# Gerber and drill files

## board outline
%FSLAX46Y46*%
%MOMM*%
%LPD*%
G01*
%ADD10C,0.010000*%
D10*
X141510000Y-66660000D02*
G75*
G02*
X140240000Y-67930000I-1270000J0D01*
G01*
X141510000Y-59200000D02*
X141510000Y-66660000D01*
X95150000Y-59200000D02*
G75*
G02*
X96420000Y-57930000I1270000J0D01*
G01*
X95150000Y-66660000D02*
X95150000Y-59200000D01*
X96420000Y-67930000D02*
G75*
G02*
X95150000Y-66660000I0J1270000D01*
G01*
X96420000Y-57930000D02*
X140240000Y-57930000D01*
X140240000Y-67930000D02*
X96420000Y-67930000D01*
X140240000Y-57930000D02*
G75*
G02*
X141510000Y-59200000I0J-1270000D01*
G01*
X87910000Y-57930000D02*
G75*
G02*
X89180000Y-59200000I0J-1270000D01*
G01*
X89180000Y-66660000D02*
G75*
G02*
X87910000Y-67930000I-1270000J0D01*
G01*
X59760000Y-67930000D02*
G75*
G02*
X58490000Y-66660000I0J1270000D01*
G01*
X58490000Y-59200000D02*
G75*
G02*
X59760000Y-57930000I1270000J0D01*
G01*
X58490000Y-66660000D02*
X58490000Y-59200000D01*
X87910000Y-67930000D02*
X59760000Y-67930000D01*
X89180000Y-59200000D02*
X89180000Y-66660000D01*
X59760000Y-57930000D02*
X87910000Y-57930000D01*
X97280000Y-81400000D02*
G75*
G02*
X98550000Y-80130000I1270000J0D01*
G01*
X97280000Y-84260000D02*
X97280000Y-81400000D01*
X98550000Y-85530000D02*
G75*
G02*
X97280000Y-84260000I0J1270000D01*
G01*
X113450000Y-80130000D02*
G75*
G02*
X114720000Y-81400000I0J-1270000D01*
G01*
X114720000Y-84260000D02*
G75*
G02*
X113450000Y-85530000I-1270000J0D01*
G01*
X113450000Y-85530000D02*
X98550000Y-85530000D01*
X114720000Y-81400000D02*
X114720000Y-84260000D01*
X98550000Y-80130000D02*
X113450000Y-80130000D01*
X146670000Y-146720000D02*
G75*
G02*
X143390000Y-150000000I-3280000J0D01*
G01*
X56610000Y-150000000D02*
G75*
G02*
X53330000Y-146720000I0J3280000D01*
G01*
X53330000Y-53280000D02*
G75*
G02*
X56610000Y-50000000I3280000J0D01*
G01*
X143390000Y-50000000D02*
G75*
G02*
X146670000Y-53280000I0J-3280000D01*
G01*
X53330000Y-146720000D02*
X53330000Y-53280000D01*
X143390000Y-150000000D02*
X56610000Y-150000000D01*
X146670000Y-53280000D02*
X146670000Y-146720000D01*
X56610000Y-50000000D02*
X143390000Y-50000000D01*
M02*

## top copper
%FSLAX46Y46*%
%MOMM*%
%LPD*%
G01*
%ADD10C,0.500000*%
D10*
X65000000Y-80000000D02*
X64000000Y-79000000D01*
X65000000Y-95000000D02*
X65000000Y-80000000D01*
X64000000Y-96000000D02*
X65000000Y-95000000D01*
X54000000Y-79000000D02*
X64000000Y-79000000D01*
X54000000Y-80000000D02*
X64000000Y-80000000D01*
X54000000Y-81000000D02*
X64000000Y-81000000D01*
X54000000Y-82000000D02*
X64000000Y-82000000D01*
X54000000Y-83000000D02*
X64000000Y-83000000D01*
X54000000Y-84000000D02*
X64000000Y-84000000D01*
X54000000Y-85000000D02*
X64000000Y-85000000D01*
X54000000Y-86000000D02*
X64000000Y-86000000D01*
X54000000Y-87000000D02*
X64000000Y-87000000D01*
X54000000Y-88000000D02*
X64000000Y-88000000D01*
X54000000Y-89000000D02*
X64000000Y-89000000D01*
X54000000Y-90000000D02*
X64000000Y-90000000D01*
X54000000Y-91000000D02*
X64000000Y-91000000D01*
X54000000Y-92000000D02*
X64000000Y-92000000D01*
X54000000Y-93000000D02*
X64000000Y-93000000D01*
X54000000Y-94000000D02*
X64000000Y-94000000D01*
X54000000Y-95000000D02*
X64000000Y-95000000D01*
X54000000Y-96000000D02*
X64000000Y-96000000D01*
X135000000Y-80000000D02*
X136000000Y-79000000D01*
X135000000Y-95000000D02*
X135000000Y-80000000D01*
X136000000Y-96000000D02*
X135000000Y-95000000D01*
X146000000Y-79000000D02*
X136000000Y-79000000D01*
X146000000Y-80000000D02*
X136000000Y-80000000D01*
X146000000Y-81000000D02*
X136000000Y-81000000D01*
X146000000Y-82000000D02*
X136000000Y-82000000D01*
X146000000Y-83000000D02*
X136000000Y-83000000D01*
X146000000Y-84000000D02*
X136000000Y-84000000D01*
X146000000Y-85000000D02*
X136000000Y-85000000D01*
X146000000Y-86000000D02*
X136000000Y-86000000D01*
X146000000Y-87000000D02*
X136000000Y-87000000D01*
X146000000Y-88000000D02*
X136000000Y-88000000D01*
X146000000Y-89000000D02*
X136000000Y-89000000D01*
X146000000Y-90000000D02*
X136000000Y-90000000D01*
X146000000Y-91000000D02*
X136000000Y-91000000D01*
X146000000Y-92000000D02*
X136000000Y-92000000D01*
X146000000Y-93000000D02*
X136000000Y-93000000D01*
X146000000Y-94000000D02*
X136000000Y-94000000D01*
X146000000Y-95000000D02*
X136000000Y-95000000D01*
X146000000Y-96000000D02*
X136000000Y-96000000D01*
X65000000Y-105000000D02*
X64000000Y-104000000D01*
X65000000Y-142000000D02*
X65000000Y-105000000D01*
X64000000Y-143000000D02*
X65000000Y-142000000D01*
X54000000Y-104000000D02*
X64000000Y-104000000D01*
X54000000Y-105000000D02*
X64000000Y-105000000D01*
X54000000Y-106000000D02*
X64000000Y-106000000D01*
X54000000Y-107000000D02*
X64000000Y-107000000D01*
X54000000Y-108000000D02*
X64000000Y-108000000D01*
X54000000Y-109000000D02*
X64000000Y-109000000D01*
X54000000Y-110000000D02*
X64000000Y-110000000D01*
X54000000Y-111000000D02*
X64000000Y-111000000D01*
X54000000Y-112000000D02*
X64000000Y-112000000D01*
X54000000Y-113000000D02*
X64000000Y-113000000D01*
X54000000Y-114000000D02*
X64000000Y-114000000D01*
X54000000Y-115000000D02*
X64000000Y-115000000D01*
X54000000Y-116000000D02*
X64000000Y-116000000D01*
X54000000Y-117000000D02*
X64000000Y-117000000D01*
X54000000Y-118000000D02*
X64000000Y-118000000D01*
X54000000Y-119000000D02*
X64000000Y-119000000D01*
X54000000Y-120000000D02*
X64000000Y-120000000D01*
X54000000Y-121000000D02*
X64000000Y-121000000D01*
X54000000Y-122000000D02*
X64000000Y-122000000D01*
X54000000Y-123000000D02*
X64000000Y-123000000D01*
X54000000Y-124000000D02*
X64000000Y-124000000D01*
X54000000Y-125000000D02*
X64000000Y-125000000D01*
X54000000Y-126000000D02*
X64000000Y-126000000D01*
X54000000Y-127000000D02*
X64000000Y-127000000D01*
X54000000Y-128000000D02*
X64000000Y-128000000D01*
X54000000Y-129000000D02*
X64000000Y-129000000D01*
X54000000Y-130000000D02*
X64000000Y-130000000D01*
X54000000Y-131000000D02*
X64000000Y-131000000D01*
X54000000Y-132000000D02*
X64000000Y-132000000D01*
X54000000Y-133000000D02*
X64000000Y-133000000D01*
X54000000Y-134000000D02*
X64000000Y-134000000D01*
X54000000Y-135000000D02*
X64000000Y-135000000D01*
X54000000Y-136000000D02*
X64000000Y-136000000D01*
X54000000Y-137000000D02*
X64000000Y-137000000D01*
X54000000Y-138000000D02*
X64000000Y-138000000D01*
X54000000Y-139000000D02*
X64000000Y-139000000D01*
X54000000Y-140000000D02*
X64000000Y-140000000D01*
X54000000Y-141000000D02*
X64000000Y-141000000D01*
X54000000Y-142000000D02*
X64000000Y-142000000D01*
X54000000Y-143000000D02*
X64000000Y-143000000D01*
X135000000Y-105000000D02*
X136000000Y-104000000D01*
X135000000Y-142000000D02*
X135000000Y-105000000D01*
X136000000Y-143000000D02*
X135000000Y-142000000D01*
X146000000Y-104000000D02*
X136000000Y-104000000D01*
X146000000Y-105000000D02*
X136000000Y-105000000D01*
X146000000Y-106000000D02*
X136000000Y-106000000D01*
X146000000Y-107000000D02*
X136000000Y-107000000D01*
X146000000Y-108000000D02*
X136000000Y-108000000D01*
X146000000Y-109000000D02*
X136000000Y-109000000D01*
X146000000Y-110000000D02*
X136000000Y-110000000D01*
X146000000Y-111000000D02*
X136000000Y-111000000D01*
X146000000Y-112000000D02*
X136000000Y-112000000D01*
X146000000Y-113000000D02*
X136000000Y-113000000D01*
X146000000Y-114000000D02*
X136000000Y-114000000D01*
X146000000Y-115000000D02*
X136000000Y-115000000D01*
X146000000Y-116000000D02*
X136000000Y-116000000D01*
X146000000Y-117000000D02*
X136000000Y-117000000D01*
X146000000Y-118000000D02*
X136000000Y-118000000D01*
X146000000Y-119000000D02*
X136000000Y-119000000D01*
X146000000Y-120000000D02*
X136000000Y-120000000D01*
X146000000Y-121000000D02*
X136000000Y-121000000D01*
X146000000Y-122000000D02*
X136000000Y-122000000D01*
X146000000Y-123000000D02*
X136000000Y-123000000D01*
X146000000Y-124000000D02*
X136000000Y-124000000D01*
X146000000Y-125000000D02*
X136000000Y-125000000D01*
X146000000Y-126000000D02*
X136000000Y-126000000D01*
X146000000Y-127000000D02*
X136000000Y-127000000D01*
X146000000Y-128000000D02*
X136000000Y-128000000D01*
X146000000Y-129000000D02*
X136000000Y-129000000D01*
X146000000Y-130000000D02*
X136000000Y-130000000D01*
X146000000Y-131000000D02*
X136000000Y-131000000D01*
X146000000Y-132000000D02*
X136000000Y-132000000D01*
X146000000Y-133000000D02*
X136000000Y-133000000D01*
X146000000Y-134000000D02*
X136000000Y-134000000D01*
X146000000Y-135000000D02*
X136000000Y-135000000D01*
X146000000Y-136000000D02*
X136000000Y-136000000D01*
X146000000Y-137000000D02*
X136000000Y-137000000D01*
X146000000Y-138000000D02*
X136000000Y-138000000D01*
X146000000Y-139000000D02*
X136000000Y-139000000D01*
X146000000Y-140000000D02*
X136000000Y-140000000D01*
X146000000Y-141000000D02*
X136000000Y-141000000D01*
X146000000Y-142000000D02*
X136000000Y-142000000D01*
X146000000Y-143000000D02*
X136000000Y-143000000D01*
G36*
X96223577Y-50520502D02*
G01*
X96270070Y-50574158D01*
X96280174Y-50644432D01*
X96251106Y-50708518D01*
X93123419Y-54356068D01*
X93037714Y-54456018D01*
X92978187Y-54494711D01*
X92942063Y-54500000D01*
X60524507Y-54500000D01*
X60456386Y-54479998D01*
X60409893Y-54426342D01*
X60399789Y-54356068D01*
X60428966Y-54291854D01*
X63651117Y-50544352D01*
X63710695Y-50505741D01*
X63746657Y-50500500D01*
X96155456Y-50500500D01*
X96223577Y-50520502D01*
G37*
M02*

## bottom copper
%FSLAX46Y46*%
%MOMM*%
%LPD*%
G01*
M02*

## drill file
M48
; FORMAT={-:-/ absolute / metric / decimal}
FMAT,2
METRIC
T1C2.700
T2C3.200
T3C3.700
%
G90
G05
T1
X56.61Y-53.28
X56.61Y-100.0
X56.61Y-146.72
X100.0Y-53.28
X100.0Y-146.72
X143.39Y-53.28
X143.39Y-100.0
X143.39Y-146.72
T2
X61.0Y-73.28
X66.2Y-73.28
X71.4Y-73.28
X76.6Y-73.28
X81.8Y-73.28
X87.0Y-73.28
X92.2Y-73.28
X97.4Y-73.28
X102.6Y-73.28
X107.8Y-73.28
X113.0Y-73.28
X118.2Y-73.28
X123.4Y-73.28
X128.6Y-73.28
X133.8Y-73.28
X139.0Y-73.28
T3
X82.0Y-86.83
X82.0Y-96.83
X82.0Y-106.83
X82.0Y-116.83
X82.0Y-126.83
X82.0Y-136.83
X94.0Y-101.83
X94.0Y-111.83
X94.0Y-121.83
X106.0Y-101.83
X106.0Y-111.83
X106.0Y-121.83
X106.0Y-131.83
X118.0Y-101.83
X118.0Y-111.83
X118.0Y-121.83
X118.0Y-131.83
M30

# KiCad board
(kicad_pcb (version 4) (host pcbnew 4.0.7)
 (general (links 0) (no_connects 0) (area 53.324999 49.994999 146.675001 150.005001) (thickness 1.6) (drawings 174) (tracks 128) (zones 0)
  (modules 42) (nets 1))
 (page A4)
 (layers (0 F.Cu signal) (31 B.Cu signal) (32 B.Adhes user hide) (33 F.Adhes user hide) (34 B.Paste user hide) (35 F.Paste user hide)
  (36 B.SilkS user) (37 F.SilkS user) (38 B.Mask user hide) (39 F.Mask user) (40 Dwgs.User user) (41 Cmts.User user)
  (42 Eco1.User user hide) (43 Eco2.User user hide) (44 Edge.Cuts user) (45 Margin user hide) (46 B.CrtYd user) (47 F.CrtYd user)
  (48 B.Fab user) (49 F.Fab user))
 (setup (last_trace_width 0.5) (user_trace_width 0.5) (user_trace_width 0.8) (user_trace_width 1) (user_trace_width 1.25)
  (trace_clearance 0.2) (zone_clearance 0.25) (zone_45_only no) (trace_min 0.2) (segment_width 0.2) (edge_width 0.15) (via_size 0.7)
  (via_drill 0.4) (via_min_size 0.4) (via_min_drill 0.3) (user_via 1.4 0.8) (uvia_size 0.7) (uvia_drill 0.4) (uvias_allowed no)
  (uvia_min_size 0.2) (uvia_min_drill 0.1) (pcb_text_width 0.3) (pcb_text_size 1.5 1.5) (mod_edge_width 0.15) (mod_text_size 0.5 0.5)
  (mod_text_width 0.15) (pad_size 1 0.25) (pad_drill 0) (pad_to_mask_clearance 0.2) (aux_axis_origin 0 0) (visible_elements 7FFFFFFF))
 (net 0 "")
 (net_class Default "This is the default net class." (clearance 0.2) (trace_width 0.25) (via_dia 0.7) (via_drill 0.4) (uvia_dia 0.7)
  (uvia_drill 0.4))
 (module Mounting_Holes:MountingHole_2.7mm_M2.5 (layer F.Cu) (at 143.39 146.72)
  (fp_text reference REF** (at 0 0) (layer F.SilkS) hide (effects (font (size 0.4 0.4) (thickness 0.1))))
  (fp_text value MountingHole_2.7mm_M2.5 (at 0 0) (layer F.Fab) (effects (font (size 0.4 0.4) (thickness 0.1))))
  (pad 1 np_thru_hole circle (at 0 0) (size 2.7 2.7) (drill 2.7) (layers *.Cu *.Mask)))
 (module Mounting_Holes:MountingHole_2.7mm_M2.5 (layer F.Cu) (at 100 146.72)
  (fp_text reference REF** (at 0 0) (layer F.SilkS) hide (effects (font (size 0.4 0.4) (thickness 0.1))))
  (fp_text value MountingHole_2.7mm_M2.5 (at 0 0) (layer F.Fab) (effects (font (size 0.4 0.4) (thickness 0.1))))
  (pad 1 np_thru_hole circle (at 0 0) (size 2.7 2.7) (drill 2.7) (layers *.Cu *.Mask)))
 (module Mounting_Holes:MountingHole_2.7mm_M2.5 (layer F.Cu) (at 56.61 146.72)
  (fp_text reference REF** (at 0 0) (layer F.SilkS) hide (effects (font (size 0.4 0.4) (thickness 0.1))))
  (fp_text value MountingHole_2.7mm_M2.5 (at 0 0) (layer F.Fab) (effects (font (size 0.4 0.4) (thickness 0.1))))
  (pad 1 np_thru_hole circle (at 0 0) (size 2.7 2.7) (drill 2.7) (layers *.Cu *.Mask)))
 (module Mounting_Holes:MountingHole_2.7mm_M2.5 (layer F.Cu) (at 143.39 100)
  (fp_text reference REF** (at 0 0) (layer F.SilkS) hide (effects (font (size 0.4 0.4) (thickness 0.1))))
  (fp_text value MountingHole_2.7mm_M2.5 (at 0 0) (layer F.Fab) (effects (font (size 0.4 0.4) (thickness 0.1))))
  (pad 1 np_thru_hole circle (at 0 0) (size 2.7 2.7) (drill 2.7) (layers *.Cu *.Mask)))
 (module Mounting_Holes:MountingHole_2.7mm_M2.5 (layer F.Cu) (at 56.61 100)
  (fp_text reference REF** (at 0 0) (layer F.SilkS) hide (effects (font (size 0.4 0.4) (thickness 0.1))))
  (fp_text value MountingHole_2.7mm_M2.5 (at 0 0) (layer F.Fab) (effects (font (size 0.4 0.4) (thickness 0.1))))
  (pad 1 np_thru_hole circle (at 0 0) (size 2.7 2.7) (drill 2.7) (layers *.Cu *.Mask)))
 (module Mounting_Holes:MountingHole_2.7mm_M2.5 (layer F.Cu) (at 143.39 53.28)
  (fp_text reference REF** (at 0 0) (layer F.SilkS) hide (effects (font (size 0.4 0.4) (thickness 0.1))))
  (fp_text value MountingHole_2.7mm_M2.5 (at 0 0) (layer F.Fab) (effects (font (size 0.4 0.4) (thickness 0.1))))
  (pad 1 np_thru_hole circle (at 0 0) (size 2.7 2.7) (drill 2.7) (layers *.Cu *.Mask)))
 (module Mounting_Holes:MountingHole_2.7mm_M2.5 (layer F.Cu) (at 100 53.28)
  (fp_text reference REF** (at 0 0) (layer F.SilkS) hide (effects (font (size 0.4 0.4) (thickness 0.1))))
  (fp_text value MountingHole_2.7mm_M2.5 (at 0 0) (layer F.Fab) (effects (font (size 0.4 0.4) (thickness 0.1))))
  (pad 1 np_thru_hole circle (at 0 0) (size 2.7 2.7) (drill 2.7) (layers *.Cu *.Mask)))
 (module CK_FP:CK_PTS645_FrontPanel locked (layer F.Cu) (at 82 136.83)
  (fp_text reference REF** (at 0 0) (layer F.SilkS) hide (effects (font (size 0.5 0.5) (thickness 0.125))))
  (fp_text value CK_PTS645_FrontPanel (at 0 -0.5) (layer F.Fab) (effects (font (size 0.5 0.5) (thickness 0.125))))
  (pad "" np_thru_hole circle (at 0 0) (size 3.7 3.7) (drill 3.7) (layers *.Cu *.Mask)))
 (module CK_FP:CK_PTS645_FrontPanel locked (layer F.Cu) (at 82 86.83)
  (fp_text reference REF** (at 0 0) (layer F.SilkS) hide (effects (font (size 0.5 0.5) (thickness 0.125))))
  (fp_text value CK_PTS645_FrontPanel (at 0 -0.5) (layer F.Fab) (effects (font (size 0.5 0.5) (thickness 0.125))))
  (pad "" np_thru_hole circle (at 0 0) (size 3.7 3.7) (drill 3.7) (layers *.Cu *.Mask)))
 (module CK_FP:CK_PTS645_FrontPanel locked (layer F.Cu) (at 82 96.83)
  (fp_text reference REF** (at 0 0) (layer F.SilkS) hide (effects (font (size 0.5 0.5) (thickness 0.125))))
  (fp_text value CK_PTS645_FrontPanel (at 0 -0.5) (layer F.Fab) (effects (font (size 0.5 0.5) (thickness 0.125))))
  (pad "" np_thru_hole circle (at 0 0) (size 3.7 3.7) (drill 3.7) (layers *.Cu *.Mask)))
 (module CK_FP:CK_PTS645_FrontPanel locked (layer F.Cu) (at 82 106.83)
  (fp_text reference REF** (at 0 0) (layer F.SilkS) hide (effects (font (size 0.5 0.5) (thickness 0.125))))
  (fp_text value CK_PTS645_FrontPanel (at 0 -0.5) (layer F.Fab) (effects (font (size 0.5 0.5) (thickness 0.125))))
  (pad "" np_thru_hole circle (at 0 0) (size 3.7 3.7) (drill 3.7) (layers *.Cu *.Mask)))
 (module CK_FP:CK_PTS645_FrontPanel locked (layer F.Cu) (at 82 116.83)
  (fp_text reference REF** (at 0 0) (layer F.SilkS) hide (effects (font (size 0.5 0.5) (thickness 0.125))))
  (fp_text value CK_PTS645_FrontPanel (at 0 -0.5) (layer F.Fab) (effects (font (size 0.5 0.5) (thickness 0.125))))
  (pad "" np_thru_hole circle (at 0 0) (size 3.7 3.7) (drill 3.7) (layers *.Cu *.Mask)))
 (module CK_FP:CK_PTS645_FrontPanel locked (layer F.Cu) (at 82 126.83)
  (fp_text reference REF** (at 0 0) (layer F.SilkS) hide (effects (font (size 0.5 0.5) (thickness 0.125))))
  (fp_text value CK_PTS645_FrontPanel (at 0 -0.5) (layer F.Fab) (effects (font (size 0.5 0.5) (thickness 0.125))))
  (pad "" np_thru_hole circle (at 0 0) (size 3.7 3.7) (drill 3.7) (layers *.Cu *.Mask)))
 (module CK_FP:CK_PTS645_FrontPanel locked (layer F.Cu) (at 106 131.83)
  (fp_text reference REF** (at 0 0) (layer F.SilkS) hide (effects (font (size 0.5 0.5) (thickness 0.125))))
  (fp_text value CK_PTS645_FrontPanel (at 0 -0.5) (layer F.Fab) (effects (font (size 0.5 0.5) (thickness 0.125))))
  (pad "" np_thru_hole circle (at 0 0) (size 3.7 3.7) (drill 3.7) (layers *.Cu *.Mask)))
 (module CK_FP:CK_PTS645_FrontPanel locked (layer F.Cu) (at 118 131.83)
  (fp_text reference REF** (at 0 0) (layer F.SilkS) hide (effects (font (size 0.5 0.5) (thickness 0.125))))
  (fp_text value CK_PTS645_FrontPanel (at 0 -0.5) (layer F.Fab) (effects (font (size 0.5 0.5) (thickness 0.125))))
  (pad "" np_thru_hole circle (at 0 0) (size 3.7 3.7) (drill 3.7) (layers *.Cu *.Mask)))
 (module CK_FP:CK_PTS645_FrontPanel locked (layer F.Cu) (at 94 121.83)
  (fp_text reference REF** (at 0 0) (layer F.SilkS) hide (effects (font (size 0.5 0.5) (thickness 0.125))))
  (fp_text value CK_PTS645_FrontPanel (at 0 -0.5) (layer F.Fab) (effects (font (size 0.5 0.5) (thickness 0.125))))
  (pad "" np_thru_hole circle (at 0 0) (size 3.7 3.7) (drill 3.7) (layers *.Cu *.Mask)))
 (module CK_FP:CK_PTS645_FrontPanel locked (layer F.Cu) (at 106 121.83)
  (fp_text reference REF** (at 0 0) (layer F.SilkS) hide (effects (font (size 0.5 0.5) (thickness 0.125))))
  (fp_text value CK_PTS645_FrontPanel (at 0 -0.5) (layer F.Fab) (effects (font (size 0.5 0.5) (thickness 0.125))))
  (pad "" np_thru_hole circle (at 0 0) (size 3.7 3.7) (drill 3.7) (layers *.Cu *.Mask)))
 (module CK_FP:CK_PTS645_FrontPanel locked (layer F.Cu) (at 118 121.83)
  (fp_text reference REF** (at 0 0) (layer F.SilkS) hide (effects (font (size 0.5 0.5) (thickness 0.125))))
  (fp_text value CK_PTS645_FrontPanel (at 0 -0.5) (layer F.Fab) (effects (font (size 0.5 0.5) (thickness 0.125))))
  (pad "" np_thru_hole circle (at 0 0) (size 3.7 3.7) (drill 3.7) (layers *.Cu *.Mask)))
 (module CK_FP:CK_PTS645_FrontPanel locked (layer F.Cu) (at 94 111.83)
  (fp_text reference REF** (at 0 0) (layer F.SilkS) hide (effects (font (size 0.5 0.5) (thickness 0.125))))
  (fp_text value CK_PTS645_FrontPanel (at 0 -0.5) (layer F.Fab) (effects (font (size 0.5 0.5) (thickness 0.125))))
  (pad "" np_thru_hole circle (at 0 0) (size 3.7 3.7) (drill 3.7) (layers *.Cu *.Mask)))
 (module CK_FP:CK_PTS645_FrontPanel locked (layer F.Cu) (at 106 111.83)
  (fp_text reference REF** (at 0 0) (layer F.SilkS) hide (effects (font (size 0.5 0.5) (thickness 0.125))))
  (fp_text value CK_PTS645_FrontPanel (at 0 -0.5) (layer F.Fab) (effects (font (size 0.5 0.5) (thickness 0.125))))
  (pad "" np_thru_hole circle (at 0 0) (size 3.7 3.7) (drill 3.7) (layers *.Cu *.Mask)))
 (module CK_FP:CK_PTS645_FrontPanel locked (layer F.Cu) (at 118 111.83)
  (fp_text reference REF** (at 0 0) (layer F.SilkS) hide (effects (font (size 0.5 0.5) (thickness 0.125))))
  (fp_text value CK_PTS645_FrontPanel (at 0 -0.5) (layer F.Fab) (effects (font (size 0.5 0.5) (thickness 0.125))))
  (pad "" np_thru_hole circle (at 0 0) (size 3.7 3.7) (drill 3.7) (layers *.Cu *.Mask)))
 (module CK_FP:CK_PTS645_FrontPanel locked (layer F.Cu) (at 94 101.83)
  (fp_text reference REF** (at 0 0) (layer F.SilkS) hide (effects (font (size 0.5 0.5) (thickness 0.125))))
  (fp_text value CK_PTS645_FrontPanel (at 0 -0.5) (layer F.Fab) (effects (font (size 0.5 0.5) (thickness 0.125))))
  (pad "" np_thru_hole circle (at 0 0) (size 3.7 3.7) (drill 3.7) (layers *.Cu *.Mask)))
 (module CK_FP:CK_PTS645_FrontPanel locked (layer F.Cu) (at 106 101.83)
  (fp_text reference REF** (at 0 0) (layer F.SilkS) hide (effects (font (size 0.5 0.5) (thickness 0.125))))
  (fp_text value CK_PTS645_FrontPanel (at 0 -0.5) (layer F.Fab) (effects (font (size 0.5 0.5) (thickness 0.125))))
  (pad "" np_thru_hole circle (at 0 0) (size 3.7 3.7) (drill 3.7) (layers *.Cu *.Mask)))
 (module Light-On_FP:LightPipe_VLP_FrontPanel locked (layer F.Cu) (at 61 73.28)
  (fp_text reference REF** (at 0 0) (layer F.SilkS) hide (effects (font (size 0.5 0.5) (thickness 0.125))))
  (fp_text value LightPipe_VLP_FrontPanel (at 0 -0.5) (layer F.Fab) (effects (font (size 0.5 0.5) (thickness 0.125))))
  (pad "" np_thru_hole circle (at 0 0) (size 3.2 3.2) (drill 3.2) (layers *.Cu *.Mask)))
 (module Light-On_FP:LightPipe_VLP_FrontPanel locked (layer F.Cu) (at 66.2 73.28)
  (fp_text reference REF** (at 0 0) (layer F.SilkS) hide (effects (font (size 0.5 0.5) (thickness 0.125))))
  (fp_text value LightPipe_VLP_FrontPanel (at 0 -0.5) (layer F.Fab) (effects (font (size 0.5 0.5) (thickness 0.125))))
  (pad "" np_thru_hole circle (at 0 0) (size 3.2 3.2) (drill 3.2) (layers *.Cu *.Mask)))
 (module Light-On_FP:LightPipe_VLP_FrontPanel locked (layer F.Cu) (at 71.4 73.28)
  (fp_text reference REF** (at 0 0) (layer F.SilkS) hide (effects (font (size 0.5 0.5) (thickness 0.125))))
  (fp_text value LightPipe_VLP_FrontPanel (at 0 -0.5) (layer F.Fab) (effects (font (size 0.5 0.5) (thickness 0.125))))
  (pad "" np_thru_hole circle (at 0 0) (size 3.2 3.2) (drill 3.2) (layers *.Cu *.Mask)))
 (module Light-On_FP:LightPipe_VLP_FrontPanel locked (layer F.Cu) (at 76.6 73.28)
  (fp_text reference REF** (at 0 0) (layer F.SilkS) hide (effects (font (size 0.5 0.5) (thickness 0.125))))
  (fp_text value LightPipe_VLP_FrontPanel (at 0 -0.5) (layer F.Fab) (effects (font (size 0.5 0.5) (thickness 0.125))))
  (pad "" np_thru_hole circle (at 0 0) (size 3.2 3.2) (drill 3.2) (layers *.Cu *.Mask)))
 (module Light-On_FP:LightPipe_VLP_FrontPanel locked (layer F.Cu) (at 81.8 73.28)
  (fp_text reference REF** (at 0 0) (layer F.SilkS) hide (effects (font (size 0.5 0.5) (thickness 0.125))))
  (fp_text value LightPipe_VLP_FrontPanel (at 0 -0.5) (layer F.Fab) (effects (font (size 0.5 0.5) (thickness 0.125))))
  (pad "" np_thru_hole circle (at 0 0) (size 3.2 3.2) (drill 3.2) (layers *.Cu *.Mask)))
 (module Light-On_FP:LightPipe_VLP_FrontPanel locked (layer F.Cu) (at 87 73.28)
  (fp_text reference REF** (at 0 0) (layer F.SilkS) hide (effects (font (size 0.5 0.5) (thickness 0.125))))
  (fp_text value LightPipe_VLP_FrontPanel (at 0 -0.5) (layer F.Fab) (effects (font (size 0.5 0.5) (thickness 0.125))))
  (pad "" np_thru_hole circle (at 0 0) (size 3.2 3.2) (drill 3.2) (layers *.Cu *.Mask)))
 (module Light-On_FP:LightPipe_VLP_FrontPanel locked (layer F.Cu) (at 92.2 73.28)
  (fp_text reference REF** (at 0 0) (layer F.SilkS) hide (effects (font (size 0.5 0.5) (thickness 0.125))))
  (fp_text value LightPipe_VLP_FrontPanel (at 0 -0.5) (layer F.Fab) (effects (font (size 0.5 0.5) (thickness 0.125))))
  (pad "" np_thru_hole circle (at 0 0) (size 3.2 3.2) (drill 3.2) (layers *.Cu *.Mask)))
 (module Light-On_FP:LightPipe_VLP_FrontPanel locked (layer F.Cu) (at 97.4 73.28)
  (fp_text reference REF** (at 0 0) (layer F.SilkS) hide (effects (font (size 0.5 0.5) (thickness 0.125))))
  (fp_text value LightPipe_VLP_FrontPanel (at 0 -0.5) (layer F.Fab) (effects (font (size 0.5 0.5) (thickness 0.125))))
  (pad "" np_thru_hole circle (at 0 0) (size 3.2 3.2) (drill 3.2) (layers *.Cu *.Mask)))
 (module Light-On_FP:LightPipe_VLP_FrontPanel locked (layer F.Cu) (at 102.6 73.28)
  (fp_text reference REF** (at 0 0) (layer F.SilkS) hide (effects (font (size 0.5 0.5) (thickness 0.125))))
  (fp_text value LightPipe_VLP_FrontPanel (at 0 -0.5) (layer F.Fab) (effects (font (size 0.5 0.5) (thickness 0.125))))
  (pad "" np_thru_hole circle (at 0 0) (size 3.2 3.2) (drill 3.2) (layers *.Cu *.Mask)))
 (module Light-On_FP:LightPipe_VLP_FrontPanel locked (layer F.Cu) (at 107.8 73.28)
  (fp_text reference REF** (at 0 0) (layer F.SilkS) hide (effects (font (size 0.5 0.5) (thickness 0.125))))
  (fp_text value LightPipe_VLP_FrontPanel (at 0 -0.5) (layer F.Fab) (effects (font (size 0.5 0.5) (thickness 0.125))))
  (pad "" np_thru_hole circle (at 0 0) (size 3.2 3.2) (drill 3.2) (layers *.Cu *.Mask)))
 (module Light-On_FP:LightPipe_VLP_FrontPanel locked (layer F.Cu) (at 113 73.28)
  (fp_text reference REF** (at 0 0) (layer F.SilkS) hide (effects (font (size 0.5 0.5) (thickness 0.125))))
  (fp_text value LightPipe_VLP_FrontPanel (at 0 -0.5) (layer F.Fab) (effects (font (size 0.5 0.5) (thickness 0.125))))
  (pad "" np_thru_hole circle (at 0 0) (size 3.2 3.2) (drill 3.2) (layers *.Cu *.Mask)))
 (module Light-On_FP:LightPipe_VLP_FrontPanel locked (layer F.Cu) (at 118.2 73.28)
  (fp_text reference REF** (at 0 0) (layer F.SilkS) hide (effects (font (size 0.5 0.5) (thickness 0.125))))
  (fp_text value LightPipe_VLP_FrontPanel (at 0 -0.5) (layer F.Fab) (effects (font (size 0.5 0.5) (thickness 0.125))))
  (pad "" np_thru_hole circle (at 0 0) (size 3.2 3.2) (drill 3.2) (layers *.Cu *.Mask)))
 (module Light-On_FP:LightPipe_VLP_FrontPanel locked (layer F.Cu) (at 123.4 73.28)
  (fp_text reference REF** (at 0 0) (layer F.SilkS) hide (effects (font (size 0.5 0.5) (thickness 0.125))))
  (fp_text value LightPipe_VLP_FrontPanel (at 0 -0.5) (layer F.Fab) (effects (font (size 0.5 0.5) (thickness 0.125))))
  (pad "" np_thru_hole circle (at 0 0) (size 3.2 3.2) (drill 3.2) (layers *.Cu *.Mask)))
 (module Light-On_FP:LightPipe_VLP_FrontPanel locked (layer F.Cu) (at 128.6 73.28)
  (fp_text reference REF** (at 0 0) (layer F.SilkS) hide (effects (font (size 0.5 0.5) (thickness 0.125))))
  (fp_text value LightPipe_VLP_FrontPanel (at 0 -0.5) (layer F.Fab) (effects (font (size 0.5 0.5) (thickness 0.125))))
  (pad "" np_thru_hole circle (at 0 0) (size 3.2 3.2) (drill 3.2) (layers *.Cu *.Mask)))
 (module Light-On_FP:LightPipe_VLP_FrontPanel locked (layer F.Cu) (at 133.8 73.28)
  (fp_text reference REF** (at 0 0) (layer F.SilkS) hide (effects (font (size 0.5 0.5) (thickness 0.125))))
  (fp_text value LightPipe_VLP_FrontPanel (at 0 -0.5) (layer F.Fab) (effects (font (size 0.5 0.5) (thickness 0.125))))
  (pad "" np_thru_hole circle (at 0 0) (size 3.2 3.2) (drill 3.2) (layers *.Cu *.Mask)))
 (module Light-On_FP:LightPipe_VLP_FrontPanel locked (layer F.Cu) (at 139 73.28)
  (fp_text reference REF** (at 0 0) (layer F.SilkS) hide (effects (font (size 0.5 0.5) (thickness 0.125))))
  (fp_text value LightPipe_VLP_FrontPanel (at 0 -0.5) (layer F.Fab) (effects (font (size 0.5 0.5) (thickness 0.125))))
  (pad "" np_thru_hole circle (at 0 0) (size 3.2 3.2) (drill 3.2) (layers *.Cu *.Mask)))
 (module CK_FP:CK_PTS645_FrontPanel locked (layer F.Cu) (at 118 101.83)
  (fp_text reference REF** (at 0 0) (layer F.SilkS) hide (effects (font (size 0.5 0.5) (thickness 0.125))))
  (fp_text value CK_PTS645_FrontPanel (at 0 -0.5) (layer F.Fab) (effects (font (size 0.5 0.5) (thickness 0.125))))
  (pad "" np_thru_hole circle (at 0 0) (size 3.7 3.7) (drill 3.7) (layers *.Cu *.Mask)))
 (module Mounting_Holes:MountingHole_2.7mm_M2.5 (layer F.Cu) (at 56.61 53.28)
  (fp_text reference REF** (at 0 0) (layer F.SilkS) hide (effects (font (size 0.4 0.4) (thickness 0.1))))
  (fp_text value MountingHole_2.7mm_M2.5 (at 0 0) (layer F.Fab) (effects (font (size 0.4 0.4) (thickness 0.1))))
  (pad 1 np_thru_hole circle (at 0 0) (size 2.7 2.7) (drill 2.7) (layers *.Cu *.Mask)))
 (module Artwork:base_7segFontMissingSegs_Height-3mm (layer F.Cu) (at 72.19 52.37)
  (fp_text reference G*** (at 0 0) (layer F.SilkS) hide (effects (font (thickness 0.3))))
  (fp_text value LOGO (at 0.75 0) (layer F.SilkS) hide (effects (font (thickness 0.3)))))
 (gr_arc (start 140.24 66.66) (end 141.51 66.66) (angle 90) (layer Edge.Cuts) (width 0.01))
 (gr_line (start 141.51 59.2) (end 141.51 66.66) (layer Edge.Cuts) (width 0.01))
 (gr_arc (start 96.42 59.2) (end 95.15 59.2) (angle 90) (layer Edge.Cuts) (width 0.01))
 (gr_line (start 95.15 66.66) (end 95.15 59.2) (layer Edge.Cuts) (width 0.01))
 (gr_arc (start 96.42 66.66) (end 96.42 67.93) (angle 90) (layer Edge.Cuts) (width 0.01))
 (gr_line (start 96.42 57.93) (end 140.24 57.93) (layer Edge.Cuts) (width 0.01))
 (gr_line (start 140.24 67.93) (end 96.42 67.93) (layer Edge.Cuts) (width 0.01))
 (gr_arc (start 140.24 59.2) (end 140.24 57.93) (angle 90) (layer Edge.Cuts) (width 0.01))
 (gr_arc (start 87.91 59.2) (end 87.91 57.93) (angle 90) (layer Edge.Cuts) (width 0.01))
 (gr_arc (start 87.91 66.66) (end 89.18 66.66) (angle 90) (layer Edge.Cuts) (width 0.01))
 (gr_arc (start 59.76 66.66) (end 59.76 67.93) (angle 90) (layer Edge.Cuts) (width 0.01))
 (gr_arc (start 59.76 59.2) (end 58.49 59.2) (angle 90) (layer Edge.Cuts) (width 0.01))
 (gr_line (start 58.49 66.66) (end 58.49 59.2) (layer Edge.Cuts) (width 0.01))
 (gr_line (start 87.91 67.93) (end 59.76 67.93) (layer Edge.Cuts) (width 0.01))
 (gr_line (start 89.18 59.2) (end 89.18 66.66) (layer Edge.Cuts) (width 0.01))
 (gr_line (start 59.76 57.93) (end 87.91 57.93) (layer Edge.Cuts) (width 0.01))
 (gr_arc (start 98.55 81.4) (end 97.28 81.4) (angle 90) (layer Edge.Cuts) (width 0.01))
 (gr_line (start 97.28 84.26) (end 97.28 81.4) (layer Edge.Cuts) (width 0.01))
 (gr_arc (start 98.55 84.26) (end 98.55 85.53) (angle 90) (layer Edge.Cuts) (width 0.01))
 (gr_arc (start 113.45 81.4) (end 113.45 80.13) (angle 90) (layer Edge.Cuts) (width 0.01))
 (gr_arc (start 113.45 84.26) (end 114.72 84.26) (angle 90) (layer Edge.Cuts) (width 0.01))
 (gr_line (start 113.45 85.53) (end 98.55 85.53) (layer Edge.Cuts) (width 0.01))
 (gr_line (start 114.72 81.4) (end 114.72 84.26) (layer Edge.Cuts) (width 0.01))
 (gr_line (start 98.55 80.13) (end 113.45 80.13) (layer Edge.Cuts) (width 0.01))
 (gr_arc (start 143.39 146.72) (end 146.67 146.72) (angle 90) (layer Edge.Cuts) (width 0.01))
 (gr_arc (start 56.61 146.72) (end 56.61 150) (angle 90) (layer Edge.Cuts) (width 0.01))
 (gr_arc (start 56.61 53.28) (end 53.33 53.28) (angle 90) (layer Edge.Cuts) (width 0.01))
 (gr_arc (start 143.39 53.28) (end 143.39 50) (angle 90) (layer Edge.Cuts) (width 0.01))
 (gr_line (start 53.33 146.72) (end 53.33 53.28) (layer Edge.Cuts) (width 0.01))
 (gr_line (start 143.39 150) (end 56.61 150) (layer Edge.Cuts) (width 0.01))
 (gr_line (start 146.67 53.28) (end 146.67 146.72) (layer Edge.Cuts) (width 0.01))
 (gr_line (start 56.61 50) (end 143.39 50) (layer Edge.Cuts) (width 0.01))
 (segment (start 65 80) (end 64 79) (width 0.5) (layer F.Cu) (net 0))
 (segment (start 65 95) (end 65 80) (width 0.5) (layer F.Cu) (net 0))
 (segment (start 64 96) (end 65 95) (width 0.5) (layer F.Cu) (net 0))
 (segment (start 54 79) (end 64 79) (width 0.5) (layer F.Cu) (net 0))
 (segment (start 54 80) (end 64 80) (width 0.5) (layer F.Cu) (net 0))
 (segment (start 54 81) (end 64 81) (width 0.5) (layer F.Cu) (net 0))
 (segment (start 54 82) (end 64 82) (width 0.5) (layer F.Cu) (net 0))
 (segment (start 54 83) (end 64 83) (width 0.5) (layer F.Cu) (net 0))
 (segment (start 54 84) (end 64 84) (width 0.5) (layer F.Cu) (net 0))
 (segment (start 54 85) (end 64 85) (width 0.5) (layer F.Cu) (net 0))
 (segment (start 54 86) (end 64 86) (width 0.5) (layer F.Cu) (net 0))
 (segment (start 54 87) (end 64 87) (width 0.5) (layer F.Cu) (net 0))
 (segment (start 54 88) (end 64 88) (width 0.5) (layer F.Cu) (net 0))
 (segment (start 54 89) (end 64 89) (width 0.5) (layer F.Cu) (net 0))
 (segment (start 54 90) (end 64 90) (width 0.5) (layer F.Cu) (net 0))
 (segment (start 54 91) (end 64 91) (width 0.5) (layer F.Cu) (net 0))
 (segment (start 54 92) (end 64 92) (width 0.5) (layer F.Cu) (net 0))
 (segment (start 54 93) (end 64 93) (width 0.5) (layer F.Cu) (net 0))
 (segment (start 54 94) (end 64 94) (width 0.5) (layer F.Cu) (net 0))
 (segment (start 54 95) (end 64 95) (width 0.5) (layer F.Cu) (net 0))
 (segment (start 54 96) (end 64 96) (width 0.5) (layer F.Cu) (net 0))
 (segment (start 135 80) (end 136 79) (width 0.5) (layer F.Cu) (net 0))
 (segment (start 135 95) (end 135 80) (width 0.5) (layer F.Cu) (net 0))
 (segment (start 136 96) (end 135 95) (width 0.5) (layer F.Cu) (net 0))
 (segment (start 146 79) (end 136 79) (width 0.5) (layer F.Cu) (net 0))
 (segment (start 146 80) (end 136 80) (width 0.5) (layer F.Cu) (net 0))
 (segment (start 146 81) (end 136 81) (width 0.5) (layer F.Cu) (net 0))
 (segment (start 146 82) (end 136 82) (width 0.5) (layer F.Cu) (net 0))
 (segment (start 146 83) (end 136 83) (width 0.5) (layer F.Cu) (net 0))
 (segment (start 146 84) (end 136 84) (width 0.5) (layer F.Cu) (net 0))
 (segment (start 146 85) (end 136 85) (width 0.5) (layer F.Cu) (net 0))
 (segment (start 146 86) (end 136 86) (width 0.5) (layer F.Cu) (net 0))
 (segment (start 146 87) (end 136 87) (width 0.5) (layer F.Cu) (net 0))
 (segment (start 146 88) (end 136 88) (width 0.5) (layer F.Cu) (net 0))
 (segment (start 146 89) (end 136 89) (width 0.5) (layer F.Cu) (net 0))
 (segment (start 146 90) (end 136 90) (width 0.5) (layer F.Cu) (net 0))
 (segment (start 146 91) (end 136 91) (width 0.5) (layer F.Cu) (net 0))
 (segment (start 146 92) (end 136 92) (width 0.5) (layer F.Cu) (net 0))
 (segment (start 146 93) (end 136 93) (width 0.5) (layer F.Cu) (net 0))
 (segment (start 146 94) (end 136 94) (width 0.5) (layer F.Cu) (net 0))
 (segment (start 146 95) (end 136 95) (width 0.5) (layer F.Cu) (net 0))
 (segment (start 146 96) (end 136 96) (width 0.5) (layer F.Cu) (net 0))
 (segment (start 65 105) (end 64 104) (width 0.5) (layer F.Cu) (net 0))
 (segment (start 65 142) (end 65 105) (width 0.5) (layer F.Cu) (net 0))
 (segment (start 64 143) (end 65 142) (width 0.5) (layer F.Cu) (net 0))
 (segment (start 54 104) (end 64 104) (width 0.5) (layer F.Cu) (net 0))
 (segment (start 54 105) (end 64 105) (width 0.5) (layer F.Cu) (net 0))
 (segment (start 54 106) (end 64 106) (width 0.5) (layer F.Cu) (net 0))
 (segment (start 54 107) (end 64 107) (width 0.5) (layer F.Cu) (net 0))
 (segment (start 54 108) (end 64 108) (width 0.5) (layer F.Cu) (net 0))
 (segment (start 54 109) (end 64 109) (width 0.5) (layer F.Cu) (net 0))
 (segment (start 54 110) (end 64 110) (width 0.5) (layer F.Cu) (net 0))
 (segment (start 54 111) (end 64 111) (width 0.5) (layer F.Cu) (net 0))
 (segment (start 54 112) (end 64 112) (width 0.5) (layer F.Cu) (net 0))
 (segment (start 54 113) (end 64 113) (width 0.5) (layer F.Cu) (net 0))
 (segment (start 54 114) (end 64 114) (width 0.5) (layer F.Cu) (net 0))
 (segment (start 54 115) (end 64 115) (width 0.5) (layer F.Cu) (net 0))
 (segment (start 54 116) (end 64 116) (width 0.5) (layer F.Cu) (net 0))
 (segment (start 54 117) (end 64 117) (width 0.5) (layer F.Cu) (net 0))
 (segment (start 54 118) (end 64 118) (width 0.5) (layer F.Cu) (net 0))
 (segment (start 54 119) (end 64 119) (width 0.5) (layer F.Cu) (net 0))
 (segment (start 54 120) (end 64 120) (width 0.5) (layer F.Cu) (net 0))
 (segment (start 54 121) (end 64 121) (width 0.5) (layer F.Cu) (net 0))
 (segment (start 54 122) (end 64 122) (width 0.5) (layer F.Cu) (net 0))
 (segment (start 54 123) (end 64 123) (width 0.5) (layer F.Cu) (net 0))
 (segment (start 54 124) (end 64 124) (width 0.5) (layer F.Cu) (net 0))
 (segment (start 54 125) (end 64 125) (width 0.5) (layer F.Cu) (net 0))
 (segment (start 54 126) (end 64 126) (width 0.5) (layer F.Cu) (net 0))
 (segment (start 54 127) (end 64 127) (width 0.5) (layer F.Cu) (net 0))
 (segment (start 54 128) (end 64 128) (width 0.5) (layer F.Cu) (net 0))
 (segment (start 54 129) (end 64 129) (width 0.5) (layer F.Cu) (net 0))
 (segment (start 54 130) (end 64 130) (width 0.5) (layer F.Cu) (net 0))
 (segment (start 54 131) (end 64 131) (width 0.5) (layer F.Cu) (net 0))
 (segment (start 54 132) (end 64 132) (width 0.5) (layer F.Cu) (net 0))
 (segment (start 54 133) (end 64 133) (width 0.5) (layer F.Cu) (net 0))
 (segment (start 54 134) (end 64 134) (width 0.5) (layer F.Cu) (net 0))
 (segment (start 54 135) (end 64 135) (width 0.5) (layer F.Cu) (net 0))
 (segment (start 54 136) (end 64 136) (width 0.5) (layer F.Cu) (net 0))
 (segment (start 54 137) (end 64 137) (width 0.5) (layer F.Cu) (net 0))
 (segment (start 54 138) (end 64 138) (width 0.5) (layer F.Cu) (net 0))
 (segment (start 54 139) (end 64 139) (width 0.5) (layer F.Cu) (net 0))
 (segment (start 54 140) (end 64 140) (width 0.5) (layer F.Cu) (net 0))
 (segment (start 54 141) (end 64 141) (width 0.5) (layer F.Cu) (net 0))
 (segment (start 54 142) (end 64 142) (width 0.5) (layer F.Cu) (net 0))
 (segment (start 54 143) (end 64 143) (width 0.5) (layer F.Cu) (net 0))
 (segment (start 135 105) (end 136 104) (width 0.5) (layer F.Cu) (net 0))
 (segment (start 135 142) (end 135 105) (width 0.5) (layer F.Cu) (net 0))
 (segment (start 136 143) (end 135 142) (width 0.5) (layer F.Cu) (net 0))
 (segment (start 146 104) (end 136 104) (width 0.5) (layer F.Cu) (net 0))
 (segment (start 146 105) (end 136 105) (width 0.5) (layer F.Cu) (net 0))
 (segment (start 146 106) (end 136 106) (width 0.5) (layer F.Cu) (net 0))
 (segment (start 146 107) (end 136 107) (width 0.5) (layer F.Cu) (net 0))
 (segment (start 146 108) (end 136 108) (width 0.5) (layer F.Cu) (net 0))
 (segment (start 146 109) (end 136 109) (width 0.5) (layer F.Cu) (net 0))
 (segment (start 146 110) (end 136 110) (width 0.5) (layer F.Cu) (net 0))
 (segment (start 146 111) (end 136 111) (width 0.5) (layer F.Cu) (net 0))
 (segment (start 146 112) (end 136 112) (width 0.5) (layer F.Cu) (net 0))
 (segment (start 146 113) (end 136 113) (width 0.5) (layer F.Cu) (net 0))
 (segment (start 146 114) (end 136 114) (width 0.5) (layer F.Cu) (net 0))
 (segment (start 146 115) (end 136 115) (width 0.5) (layer F.Cu) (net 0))
 (segment (start 146 116) (end 136 116) (width 0.5) (layer F.Cu) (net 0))
 (segment (start 146 117) (end 136 117) (width 0.5) (layer F.Cu) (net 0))
 (segment (start 146 118) (end 136 118) (width 0.5) (layer F.Cu) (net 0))
 (segment (start 146 119) (end 136 119) (width 0.5) (layer F.Cu) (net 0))
 (segment (start 146 120) (end 136 120) (width 0.5) (layer F.Cu) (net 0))
 (segment (start 146 121) (end 136 121) (width 0.5) (layer F.Cu) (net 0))
 (segment (start 146 122) (end 136 122) (width 0.5) (layer F.Cu) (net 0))
 (segment (start 146 123) (end 136 123) (width 0.5) (layer F.Cu) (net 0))
 (segment (start 146 124) (end 136 124) (width 0.5) (layer F.Cu) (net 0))
 (segment (start 146 125) (end 136 125) (width 0.5) (layer F.Cu) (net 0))
 (segment (start 146 126) (end 136 126) (width 0.5) (layer F.Cu) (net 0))
 (segment (start 146 127) (end 136 127) (width 0.5) (layer F.Cu) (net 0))
 (segment (start 146 128) (end 136 128) (width 0.5) (layer F.Cu) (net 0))
 (segment (start 146 129) (end 136 129) (width 0.5) (layer F.Cu) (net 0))
 (segment (start 146 130) (end 136 130) (width 0.5) (layer F.Cu) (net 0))
 (segment (start 146 131) (end 136 131) (width 0.5) (layer F.Cu) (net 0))
 (segment (start 146 132) (end 136 132) (width 0.5) (layer F.Cu) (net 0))
 (segment (start 146 133) (end 136 133) (width 0.5) (layer F.Cu) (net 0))
 (segment (start 146 134) (end 136 134) (width 0.5) (layer F.Cu) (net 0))
 (segment (start 146 135) (end 136 135) (width 0.5) (layer F.Cu) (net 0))
 (segment (start 146 136) (end 136 136) (width 0.5) (layer F.Cu) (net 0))
 (segment (start 146 137) (end 136 137) (width 0.5) (layer F.Cu) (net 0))
 (segment (start 146 138) (end 136 138) (width 0.5) (layer F.Cu) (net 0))
 (segment (start 146 139) (end 136 139) (width 0.5) (layer F.Cu) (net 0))
 (segment (start 146 140) (end 136 140) (width 0.5) (layer F.Cu) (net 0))
 (segment (start 146 141) (end 136 141) (width 0.5) (layer F.Cu) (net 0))
 (segment (start 146 142) (end 136 142) (width 0.5) (layer F.Cu) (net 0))
 (segment (start 146 143) (end 136 143) (width 0.5) (layer F.Cu) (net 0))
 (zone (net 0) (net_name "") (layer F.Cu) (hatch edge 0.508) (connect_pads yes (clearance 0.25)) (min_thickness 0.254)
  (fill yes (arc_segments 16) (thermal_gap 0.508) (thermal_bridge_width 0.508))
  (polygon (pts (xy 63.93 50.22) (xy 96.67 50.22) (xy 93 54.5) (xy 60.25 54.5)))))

